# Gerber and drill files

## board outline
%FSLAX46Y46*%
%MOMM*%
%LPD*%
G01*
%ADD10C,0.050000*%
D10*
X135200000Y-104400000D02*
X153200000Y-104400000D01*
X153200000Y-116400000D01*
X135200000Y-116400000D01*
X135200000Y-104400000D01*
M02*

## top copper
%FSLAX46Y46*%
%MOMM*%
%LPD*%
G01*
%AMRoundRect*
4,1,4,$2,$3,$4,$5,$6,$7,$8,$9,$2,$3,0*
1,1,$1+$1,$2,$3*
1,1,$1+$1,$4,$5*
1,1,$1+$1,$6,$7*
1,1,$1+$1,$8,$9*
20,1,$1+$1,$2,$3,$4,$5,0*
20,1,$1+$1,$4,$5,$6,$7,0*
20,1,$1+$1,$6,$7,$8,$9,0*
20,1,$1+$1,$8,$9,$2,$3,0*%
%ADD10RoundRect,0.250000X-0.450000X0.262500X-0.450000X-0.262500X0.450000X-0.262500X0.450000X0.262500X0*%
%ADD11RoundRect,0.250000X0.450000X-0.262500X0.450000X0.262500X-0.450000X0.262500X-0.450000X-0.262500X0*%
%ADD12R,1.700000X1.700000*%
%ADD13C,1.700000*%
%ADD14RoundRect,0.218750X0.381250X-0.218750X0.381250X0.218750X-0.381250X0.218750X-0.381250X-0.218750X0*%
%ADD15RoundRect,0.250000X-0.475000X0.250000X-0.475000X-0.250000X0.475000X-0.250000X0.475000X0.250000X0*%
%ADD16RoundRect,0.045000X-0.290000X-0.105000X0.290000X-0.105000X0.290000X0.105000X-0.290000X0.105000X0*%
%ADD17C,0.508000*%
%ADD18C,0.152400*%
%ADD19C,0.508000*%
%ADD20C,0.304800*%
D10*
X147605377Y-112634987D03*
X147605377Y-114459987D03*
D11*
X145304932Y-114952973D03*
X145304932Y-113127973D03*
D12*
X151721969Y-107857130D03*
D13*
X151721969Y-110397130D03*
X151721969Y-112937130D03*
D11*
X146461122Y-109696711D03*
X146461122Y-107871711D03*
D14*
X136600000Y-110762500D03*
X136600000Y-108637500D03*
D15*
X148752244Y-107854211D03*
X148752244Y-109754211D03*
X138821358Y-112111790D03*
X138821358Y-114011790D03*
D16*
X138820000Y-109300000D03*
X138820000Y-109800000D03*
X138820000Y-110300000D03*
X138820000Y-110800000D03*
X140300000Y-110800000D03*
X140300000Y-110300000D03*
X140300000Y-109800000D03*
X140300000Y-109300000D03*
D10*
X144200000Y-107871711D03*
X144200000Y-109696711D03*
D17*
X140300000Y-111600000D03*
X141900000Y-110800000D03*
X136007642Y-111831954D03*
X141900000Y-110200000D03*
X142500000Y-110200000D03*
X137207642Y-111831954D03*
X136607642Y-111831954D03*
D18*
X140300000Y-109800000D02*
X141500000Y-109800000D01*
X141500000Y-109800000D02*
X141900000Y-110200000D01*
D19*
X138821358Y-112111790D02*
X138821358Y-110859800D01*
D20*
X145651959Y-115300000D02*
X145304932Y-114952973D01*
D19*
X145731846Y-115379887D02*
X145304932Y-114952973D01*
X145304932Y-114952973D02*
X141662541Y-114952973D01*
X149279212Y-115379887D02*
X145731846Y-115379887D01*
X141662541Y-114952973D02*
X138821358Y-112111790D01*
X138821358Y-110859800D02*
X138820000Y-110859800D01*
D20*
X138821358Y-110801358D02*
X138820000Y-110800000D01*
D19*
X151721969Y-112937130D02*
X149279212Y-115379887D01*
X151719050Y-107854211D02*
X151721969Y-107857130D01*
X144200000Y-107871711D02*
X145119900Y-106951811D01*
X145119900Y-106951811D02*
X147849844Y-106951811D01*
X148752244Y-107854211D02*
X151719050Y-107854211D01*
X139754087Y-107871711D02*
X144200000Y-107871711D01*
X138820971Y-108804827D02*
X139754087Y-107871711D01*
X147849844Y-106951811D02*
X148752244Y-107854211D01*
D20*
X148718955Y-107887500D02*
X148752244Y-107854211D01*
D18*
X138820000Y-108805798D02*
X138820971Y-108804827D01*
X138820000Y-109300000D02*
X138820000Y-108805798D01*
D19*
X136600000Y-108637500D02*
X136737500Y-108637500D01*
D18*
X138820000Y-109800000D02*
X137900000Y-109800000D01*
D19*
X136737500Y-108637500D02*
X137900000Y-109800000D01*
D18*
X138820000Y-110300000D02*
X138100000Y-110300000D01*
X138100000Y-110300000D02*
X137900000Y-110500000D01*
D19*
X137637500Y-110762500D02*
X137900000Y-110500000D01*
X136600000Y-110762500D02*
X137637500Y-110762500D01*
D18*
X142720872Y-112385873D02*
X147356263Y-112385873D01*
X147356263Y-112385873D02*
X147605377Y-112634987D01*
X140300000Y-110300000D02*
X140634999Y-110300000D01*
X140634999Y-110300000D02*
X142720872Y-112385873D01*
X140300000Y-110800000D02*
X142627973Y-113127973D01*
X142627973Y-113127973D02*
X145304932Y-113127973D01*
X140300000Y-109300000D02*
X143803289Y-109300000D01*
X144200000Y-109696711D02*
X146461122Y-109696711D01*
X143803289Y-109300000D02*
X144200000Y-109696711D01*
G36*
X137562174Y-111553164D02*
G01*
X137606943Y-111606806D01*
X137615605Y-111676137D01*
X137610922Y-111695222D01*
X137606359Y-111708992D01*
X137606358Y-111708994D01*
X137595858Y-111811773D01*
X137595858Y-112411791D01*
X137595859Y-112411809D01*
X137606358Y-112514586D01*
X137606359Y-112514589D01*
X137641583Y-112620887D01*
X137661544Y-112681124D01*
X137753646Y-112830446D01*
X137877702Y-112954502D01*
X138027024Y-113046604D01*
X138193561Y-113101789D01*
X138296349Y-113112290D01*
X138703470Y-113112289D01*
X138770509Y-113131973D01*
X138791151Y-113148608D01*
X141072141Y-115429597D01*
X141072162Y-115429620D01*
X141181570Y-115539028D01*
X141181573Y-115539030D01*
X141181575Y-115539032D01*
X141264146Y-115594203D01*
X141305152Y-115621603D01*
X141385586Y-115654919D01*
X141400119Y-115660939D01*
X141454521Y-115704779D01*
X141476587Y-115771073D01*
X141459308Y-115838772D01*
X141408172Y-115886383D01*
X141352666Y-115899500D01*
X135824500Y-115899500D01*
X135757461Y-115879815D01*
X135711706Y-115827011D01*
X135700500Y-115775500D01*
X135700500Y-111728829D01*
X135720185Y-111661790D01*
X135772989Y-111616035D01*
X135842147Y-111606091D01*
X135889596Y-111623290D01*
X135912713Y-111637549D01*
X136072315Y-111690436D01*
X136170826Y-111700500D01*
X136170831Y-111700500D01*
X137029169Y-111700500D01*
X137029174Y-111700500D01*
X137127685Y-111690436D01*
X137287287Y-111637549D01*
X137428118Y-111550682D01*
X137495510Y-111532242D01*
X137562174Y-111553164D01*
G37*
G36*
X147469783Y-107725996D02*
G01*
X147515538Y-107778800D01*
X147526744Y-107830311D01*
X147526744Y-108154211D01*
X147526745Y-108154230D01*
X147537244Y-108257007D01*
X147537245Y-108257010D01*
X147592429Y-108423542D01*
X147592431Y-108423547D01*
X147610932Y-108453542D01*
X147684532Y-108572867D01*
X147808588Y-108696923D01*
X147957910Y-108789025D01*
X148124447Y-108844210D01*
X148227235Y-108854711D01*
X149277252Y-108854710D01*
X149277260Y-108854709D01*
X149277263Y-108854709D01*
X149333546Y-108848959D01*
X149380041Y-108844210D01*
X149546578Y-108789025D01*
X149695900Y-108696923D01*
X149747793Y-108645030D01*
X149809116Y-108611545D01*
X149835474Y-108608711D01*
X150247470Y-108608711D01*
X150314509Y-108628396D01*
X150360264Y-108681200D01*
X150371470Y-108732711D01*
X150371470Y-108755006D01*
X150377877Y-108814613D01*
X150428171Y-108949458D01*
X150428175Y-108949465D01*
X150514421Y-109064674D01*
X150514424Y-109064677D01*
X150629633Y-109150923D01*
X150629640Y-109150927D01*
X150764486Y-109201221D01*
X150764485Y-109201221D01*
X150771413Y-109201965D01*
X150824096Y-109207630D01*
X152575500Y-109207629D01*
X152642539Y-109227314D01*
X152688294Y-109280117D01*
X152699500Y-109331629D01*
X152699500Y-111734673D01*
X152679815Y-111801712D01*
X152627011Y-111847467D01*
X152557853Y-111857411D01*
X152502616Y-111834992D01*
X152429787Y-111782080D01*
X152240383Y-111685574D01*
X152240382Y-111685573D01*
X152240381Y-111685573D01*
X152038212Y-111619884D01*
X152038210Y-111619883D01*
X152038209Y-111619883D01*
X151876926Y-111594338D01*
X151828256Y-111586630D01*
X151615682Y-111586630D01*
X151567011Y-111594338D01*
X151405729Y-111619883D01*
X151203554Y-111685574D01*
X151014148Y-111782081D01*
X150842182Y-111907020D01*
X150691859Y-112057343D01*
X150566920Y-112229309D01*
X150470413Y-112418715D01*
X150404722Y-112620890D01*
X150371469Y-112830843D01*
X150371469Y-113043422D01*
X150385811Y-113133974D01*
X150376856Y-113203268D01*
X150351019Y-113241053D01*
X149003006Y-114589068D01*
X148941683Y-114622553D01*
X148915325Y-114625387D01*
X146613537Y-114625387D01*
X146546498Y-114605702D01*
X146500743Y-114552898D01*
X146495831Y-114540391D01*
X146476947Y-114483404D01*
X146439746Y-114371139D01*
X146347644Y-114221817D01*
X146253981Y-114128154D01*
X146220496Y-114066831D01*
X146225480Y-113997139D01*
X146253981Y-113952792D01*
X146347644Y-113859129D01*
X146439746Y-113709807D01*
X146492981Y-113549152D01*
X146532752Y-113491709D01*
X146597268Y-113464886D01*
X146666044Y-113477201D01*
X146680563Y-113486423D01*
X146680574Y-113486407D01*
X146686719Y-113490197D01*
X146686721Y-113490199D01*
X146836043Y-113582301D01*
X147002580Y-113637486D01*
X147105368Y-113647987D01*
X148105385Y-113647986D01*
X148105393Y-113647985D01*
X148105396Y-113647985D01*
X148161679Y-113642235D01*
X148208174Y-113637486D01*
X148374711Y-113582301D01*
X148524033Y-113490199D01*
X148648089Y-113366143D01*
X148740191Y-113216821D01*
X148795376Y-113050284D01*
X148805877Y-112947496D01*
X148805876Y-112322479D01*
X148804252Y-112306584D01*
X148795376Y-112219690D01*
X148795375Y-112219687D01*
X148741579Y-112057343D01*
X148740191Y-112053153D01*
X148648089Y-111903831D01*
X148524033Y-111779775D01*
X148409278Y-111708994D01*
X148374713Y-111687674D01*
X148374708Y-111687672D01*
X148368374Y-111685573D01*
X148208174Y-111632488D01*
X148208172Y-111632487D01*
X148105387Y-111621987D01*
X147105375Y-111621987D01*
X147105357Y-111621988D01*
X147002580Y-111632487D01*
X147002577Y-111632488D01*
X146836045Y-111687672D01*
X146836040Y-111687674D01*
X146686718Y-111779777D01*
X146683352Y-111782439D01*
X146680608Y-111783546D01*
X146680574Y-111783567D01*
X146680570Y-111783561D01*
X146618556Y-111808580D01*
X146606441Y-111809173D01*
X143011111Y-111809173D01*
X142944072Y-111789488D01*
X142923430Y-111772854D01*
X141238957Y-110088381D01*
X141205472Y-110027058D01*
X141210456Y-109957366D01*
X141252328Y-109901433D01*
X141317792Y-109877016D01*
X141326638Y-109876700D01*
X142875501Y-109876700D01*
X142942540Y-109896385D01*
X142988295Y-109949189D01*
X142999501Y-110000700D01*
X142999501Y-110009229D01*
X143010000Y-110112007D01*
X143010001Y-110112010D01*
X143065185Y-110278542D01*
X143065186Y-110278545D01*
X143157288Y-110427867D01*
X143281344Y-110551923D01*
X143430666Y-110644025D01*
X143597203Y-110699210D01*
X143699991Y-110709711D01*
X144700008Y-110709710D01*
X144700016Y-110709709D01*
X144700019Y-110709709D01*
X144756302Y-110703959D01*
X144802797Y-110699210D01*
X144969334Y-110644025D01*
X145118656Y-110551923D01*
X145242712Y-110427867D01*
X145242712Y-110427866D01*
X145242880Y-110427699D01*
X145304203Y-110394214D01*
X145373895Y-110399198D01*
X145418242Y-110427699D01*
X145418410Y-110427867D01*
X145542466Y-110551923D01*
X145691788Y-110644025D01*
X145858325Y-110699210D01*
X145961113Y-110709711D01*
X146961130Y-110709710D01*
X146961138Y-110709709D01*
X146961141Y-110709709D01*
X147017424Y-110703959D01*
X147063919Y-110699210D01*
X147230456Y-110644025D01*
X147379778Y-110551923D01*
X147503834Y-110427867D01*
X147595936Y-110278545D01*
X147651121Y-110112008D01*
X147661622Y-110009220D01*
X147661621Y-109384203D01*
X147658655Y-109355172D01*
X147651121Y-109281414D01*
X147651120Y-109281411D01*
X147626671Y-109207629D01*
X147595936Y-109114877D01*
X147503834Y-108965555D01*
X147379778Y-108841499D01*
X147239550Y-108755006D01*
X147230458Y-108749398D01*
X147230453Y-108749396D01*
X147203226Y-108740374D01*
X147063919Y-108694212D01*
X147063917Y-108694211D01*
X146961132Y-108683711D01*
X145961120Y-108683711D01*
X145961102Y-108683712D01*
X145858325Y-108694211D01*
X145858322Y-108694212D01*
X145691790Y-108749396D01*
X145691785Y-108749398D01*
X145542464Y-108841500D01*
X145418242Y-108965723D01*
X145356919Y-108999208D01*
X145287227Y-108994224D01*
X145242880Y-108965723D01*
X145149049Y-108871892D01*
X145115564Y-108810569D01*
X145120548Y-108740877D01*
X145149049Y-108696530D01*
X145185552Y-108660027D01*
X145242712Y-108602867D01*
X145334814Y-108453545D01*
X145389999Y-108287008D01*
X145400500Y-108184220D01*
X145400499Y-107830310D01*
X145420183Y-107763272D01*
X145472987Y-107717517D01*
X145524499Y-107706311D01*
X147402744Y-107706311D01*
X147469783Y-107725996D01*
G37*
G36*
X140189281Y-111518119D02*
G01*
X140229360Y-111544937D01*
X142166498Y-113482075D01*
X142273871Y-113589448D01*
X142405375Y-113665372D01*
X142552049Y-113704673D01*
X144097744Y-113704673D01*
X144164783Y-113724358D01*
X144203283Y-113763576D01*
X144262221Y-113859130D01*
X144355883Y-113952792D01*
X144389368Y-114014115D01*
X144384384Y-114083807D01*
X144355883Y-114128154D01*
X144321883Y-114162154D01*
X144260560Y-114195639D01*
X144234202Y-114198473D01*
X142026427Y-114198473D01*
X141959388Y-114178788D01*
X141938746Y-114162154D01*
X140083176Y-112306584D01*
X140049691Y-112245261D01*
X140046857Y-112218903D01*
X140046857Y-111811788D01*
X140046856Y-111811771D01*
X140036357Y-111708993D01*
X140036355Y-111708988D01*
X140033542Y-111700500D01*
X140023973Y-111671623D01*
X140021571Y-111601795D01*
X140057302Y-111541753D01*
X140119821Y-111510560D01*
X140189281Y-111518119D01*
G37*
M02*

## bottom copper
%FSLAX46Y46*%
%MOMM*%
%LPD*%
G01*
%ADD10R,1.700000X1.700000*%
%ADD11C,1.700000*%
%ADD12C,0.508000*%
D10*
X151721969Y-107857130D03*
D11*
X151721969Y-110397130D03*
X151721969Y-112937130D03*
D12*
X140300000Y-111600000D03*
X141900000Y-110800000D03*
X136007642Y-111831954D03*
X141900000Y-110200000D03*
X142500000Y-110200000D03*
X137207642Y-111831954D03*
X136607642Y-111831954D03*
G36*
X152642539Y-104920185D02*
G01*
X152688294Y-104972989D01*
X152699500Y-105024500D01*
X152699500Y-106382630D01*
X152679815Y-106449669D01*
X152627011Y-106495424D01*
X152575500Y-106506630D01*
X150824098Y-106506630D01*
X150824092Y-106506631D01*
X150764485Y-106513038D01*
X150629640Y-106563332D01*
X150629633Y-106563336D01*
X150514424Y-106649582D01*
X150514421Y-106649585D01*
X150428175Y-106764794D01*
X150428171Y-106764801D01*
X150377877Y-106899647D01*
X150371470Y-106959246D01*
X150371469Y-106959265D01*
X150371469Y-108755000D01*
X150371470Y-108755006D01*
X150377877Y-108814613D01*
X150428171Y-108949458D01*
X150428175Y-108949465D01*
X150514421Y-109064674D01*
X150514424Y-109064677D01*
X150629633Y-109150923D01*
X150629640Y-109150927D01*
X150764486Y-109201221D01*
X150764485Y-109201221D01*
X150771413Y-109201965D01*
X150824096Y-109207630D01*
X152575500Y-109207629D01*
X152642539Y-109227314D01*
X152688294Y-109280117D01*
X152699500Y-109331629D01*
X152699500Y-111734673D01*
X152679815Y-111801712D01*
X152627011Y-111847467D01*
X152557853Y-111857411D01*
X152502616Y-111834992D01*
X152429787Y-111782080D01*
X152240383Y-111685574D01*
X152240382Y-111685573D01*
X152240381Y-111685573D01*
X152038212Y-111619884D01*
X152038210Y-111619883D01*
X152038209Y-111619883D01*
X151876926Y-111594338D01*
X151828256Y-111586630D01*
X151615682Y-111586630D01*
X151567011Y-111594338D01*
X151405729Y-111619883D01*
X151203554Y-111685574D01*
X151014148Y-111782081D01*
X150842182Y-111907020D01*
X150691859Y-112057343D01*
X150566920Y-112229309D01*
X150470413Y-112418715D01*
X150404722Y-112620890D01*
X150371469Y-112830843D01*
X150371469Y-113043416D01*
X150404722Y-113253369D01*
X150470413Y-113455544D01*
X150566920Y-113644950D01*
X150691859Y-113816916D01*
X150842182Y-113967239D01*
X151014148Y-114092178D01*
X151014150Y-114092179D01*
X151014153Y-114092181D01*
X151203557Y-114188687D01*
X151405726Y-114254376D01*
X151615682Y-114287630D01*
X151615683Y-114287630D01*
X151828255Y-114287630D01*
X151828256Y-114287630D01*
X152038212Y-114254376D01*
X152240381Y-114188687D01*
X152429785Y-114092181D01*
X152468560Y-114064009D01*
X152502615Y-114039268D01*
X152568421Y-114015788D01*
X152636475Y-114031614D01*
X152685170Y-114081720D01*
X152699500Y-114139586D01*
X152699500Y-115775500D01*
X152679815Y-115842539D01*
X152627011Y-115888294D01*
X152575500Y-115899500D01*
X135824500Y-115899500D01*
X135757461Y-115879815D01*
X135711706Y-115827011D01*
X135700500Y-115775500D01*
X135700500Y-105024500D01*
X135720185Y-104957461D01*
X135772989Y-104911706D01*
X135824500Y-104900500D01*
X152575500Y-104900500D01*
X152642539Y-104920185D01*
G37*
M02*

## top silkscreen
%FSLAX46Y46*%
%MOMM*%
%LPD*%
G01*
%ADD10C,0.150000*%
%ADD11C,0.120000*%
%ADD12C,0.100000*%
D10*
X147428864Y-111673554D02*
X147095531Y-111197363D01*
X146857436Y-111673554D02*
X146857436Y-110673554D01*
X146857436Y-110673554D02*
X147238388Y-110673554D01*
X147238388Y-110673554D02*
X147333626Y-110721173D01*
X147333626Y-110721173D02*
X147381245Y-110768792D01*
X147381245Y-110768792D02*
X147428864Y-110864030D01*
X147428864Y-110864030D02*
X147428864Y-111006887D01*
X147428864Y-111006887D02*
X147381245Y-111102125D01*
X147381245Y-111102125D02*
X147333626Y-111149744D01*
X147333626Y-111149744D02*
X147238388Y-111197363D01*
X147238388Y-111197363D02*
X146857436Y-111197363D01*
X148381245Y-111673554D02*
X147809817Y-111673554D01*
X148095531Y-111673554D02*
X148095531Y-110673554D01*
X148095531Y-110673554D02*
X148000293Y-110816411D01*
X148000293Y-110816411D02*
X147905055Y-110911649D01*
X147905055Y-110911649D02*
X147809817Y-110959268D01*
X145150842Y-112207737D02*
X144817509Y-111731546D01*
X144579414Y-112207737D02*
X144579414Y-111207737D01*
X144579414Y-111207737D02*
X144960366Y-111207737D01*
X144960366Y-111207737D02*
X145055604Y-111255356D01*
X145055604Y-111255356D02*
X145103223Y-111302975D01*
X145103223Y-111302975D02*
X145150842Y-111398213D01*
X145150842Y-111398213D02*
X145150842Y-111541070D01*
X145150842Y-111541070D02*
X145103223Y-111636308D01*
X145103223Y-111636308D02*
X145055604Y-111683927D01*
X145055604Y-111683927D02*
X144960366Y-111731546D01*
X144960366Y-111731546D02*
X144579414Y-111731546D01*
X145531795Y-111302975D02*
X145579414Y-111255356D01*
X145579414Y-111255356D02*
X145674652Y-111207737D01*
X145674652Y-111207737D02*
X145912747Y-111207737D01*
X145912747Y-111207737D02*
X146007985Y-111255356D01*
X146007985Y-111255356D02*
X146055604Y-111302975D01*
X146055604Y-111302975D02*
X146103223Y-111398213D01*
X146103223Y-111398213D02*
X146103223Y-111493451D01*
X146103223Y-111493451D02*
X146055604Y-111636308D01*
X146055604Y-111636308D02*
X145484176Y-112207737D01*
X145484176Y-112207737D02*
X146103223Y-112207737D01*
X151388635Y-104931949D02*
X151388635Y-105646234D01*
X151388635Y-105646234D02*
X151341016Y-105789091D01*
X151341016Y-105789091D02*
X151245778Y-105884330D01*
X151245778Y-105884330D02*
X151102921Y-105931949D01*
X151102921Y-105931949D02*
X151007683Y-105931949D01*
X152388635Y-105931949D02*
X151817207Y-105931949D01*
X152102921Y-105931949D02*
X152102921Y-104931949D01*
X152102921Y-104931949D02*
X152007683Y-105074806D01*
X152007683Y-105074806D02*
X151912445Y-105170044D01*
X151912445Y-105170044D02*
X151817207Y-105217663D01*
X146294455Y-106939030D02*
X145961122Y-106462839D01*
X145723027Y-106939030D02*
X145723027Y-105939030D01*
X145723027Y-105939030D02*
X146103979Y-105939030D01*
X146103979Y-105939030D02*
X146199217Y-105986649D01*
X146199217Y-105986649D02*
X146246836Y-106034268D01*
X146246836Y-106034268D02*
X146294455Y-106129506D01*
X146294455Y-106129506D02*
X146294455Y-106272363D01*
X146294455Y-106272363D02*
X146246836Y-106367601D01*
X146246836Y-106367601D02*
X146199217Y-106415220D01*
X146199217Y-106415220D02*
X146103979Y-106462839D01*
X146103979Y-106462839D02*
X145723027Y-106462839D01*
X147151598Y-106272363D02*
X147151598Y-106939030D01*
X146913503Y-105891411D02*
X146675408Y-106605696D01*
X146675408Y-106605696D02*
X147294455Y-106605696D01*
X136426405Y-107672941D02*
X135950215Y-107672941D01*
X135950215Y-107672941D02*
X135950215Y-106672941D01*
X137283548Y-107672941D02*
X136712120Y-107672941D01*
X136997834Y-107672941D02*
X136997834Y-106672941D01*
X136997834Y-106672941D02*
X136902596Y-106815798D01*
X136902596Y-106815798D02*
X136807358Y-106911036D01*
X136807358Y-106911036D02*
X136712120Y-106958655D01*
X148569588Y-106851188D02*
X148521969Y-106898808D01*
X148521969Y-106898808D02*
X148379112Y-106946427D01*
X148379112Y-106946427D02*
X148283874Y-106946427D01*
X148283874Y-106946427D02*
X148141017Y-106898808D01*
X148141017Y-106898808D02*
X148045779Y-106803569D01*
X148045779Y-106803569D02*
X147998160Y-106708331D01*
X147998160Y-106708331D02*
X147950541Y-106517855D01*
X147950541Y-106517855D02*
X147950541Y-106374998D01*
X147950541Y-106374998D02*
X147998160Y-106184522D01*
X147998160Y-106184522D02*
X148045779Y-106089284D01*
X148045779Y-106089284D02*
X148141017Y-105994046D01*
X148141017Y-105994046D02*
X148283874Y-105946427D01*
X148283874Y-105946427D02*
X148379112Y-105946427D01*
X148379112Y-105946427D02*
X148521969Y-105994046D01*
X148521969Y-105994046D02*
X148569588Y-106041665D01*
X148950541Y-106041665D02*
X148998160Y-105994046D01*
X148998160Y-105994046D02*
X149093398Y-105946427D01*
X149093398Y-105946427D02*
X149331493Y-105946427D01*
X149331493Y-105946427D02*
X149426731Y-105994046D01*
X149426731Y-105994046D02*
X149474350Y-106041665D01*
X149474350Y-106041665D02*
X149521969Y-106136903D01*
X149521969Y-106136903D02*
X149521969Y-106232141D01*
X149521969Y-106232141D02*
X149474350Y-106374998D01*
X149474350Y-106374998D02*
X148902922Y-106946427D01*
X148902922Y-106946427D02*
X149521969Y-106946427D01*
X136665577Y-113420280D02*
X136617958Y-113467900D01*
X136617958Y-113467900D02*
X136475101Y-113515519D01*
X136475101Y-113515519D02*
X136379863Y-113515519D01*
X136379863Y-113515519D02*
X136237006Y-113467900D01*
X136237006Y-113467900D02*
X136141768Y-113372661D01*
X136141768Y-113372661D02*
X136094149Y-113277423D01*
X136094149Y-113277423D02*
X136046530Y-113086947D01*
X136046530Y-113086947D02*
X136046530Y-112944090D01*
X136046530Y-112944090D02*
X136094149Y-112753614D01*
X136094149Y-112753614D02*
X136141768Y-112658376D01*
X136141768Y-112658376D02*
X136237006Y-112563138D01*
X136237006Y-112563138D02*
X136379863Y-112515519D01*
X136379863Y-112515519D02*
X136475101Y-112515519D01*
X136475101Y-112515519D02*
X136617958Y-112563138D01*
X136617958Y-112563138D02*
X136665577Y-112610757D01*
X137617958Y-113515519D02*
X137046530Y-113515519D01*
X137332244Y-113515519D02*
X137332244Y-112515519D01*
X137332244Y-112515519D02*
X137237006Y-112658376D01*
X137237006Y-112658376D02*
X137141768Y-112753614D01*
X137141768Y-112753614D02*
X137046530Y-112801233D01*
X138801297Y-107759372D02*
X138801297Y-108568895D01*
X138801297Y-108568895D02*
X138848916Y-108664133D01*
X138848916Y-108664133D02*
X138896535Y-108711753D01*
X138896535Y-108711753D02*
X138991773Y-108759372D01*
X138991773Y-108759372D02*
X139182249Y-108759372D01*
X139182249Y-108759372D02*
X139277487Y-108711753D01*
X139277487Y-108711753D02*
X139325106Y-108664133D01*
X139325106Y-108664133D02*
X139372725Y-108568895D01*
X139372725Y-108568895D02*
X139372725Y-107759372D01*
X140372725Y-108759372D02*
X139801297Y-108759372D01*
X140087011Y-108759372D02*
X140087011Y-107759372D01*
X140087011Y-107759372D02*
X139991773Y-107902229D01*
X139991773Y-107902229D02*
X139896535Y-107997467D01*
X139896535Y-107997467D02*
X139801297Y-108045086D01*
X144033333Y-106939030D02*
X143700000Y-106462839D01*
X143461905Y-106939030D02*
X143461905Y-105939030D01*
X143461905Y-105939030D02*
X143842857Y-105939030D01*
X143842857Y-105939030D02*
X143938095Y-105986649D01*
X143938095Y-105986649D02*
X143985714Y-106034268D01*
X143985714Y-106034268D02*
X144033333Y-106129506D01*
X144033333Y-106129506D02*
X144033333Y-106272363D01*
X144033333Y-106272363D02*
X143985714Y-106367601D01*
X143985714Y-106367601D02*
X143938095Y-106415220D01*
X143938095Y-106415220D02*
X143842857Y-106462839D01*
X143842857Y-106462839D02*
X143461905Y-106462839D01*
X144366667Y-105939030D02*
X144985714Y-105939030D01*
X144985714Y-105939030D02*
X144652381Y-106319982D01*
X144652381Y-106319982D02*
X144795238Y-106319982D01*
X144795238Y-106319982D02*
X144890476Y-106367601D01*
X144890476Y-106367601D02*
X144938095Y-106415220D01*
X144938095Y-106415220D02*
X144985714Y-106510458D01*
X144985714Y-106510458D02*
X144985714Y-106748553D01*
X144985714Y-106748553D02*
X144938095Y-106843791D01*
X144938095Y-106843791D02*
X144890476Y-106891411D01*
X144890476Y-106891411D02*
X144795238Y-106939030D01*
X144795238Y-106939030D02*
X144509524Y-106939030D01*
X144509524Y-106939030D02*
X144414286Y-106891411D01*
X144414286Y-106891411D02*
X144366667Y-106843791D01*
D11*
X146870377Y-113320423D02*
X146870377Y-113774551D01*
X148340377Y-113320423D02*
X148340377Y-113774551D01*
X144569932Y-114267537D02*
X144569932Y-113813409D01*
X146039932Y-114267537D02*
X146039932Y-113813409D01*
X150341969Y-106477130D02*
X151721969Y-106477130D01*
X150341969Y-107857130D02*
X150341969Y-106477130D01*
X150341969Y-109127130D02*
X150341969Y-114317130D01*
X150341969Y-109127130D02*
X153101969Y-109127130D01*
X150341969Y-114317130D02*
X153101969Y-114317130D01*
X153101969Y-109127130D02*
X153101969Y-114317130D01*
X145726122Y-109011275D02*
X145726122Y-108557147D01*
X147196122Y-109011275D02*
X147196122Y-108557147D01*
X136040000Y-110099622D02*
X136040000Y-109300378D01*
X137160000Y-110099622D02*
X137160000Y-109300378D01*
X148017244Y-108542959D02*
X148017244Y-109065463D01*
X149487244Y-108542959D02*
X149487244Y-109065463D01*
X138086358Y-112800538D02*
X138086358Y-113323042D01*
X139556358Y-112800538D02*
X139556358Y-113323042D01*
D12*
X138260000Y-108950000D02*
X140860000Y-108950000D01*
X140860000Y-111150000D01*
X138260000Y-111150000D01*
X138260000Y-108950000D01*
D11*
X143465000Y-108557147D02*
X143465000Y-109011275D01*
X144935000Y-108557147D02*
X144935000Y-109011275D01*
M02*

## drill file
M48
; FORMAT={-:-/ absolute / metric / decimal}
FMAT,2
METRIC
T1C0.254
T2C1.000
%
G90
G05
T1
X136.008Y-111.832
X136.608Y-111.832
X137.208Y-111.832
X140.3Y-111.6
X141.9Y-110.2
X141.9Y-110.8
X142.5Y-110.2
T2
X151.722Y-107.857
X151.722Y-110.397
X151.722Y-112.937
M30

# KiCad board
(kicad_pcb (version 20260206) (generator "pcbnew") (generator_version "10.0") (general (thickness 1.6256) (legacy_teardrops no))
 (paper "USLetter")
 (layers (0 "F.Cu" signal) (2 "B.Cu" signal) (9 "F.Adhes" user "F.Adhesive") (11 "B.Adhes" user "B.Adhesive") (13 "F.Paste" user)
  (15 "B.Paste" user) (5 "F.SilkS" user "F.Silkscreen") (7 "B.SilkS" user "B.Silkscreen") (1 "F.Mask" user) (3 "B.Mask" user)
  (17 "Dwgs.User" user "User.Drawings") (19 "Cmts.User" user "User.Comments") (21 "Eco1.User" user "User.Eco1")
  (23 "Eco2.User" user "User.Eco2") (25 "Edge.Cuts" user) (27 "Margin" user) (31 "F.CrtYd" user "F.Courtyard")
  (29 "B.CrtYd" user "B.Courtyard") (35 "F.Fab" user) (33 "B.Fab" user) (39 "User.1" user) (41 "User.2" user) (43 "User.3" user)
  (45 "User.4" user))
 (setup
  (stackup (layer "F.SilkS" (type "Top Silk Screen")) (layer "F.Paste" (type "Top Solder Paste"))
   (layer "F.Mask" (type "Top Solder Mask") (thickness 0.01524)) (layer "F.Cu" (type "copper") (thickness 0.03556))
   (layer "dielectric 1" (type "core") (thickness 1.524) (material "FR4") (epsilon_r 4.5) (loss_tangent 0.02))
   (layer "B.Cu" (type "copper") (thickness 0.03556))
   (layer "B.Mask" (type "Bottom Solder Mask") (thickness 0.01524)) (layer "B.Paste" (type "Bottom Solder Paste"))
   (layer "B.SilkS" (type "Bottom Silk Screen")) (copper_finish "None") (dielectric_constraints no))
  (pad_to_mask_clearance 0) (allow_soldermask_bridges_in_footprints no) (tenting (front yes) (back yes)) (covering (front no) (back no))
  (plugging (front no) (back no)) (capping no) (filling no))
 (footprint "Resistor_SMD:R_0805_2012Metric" (layer "F.Cu") (at 147.605377 113.547487 -90)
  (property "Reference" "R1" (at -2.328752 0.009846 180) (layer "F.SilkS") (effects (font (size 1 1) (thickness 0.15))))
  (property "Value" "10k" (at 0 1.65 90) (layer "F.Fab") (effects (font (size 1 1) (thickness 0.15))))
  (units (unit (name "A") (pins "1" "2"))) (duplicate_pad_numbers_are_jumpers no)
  (fp_line (start -0.227064 0.735) (end 0.227064 0.735) (stroke (width 0.12) (type solid)) (layer "F.SilkS"))
  (fp_line (start -0.227064 -0.735) (end 0.227064 -0.735) (stroke (width 0.12) (type solid)) (layer "F.SilkS"))
  (pad "1" smd roundrect (at -0.9125 0 270) (size 1.025 1.4) (layers "F.Cu" "F.Mask" "F.Paste") (roundrect_rratio 0.243902)
   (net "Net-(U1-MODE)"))
  (pad "2" smd roundrect (at 0.9125 0 270) (size 1.025 1.4) (layers "F.Cu" "F.Mask" "F.Paste") (roundrect_rratio 0.243902) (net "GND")))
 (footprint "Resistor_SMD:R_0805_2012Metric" (layer "F.Cu") (at 145.304932 114.040473 90)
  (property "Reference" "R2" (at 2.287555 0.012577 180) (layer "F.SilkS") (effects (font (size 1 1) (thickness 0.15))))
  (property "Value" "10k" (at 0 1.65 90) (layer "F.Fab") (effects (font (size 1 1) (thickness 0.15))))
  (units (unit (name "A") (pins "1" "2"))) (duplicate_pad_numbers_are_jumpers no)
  (fp_line (start -0.227064 -0.735) (end 0.227064 -0.735) (stroke (width 0.12) (type solid)) (layer "F.SilkS"))
  (fp_line (start -0.227064 0.735) (end 0.227064 0.735) (stroke (width 0.12) (type solid)) (layer "F.SilkS"))
  (pad "1" smd roundrect (at -0.9125 0 90) (size 1.025 1.4) (layers "F.Cu" "F.Mask" "F.Paste") (roundrect_rratio 0.243902) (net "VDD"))
  (pad "2" smd roundrect (at 0.9125 0 90) (size 1.025 1.4) (layers "F.Cu" "F.Mask" "F.Paste") (roundrect_rratio 0.243902)
   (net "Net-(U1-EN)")))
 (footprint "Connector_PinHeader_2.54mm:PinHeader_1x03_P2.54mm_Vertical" (layer "F.Cu") (at 151.721969 107.85713)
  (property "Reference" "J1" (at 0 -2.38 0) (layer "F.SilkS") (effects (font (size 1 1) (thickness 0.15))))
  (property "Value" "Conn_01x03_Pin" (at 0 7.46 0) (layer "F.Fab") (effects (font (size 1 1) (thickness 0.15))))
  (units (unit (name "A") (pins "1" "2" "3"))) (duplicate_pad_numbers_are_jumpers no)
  (fp_line (start -1.38 -1.38) (end 0 -1.38) (stroke (width 0.12) (type solid)) (layer "F.SilkS"))
  (fp_line (start -1.38 0) (end -1.38 -1.38) (stroke (width 0.12) (type solid)) (layer "F.SilkS"))
  (fp_line (start -1.38 1.27) (end -1.38 6.46) (stroke (width 0.12) (type solid)) (layer "F.SilkS"))
  (fp_line (start -1.38 1.27) (end 1.38 1.27) (stroke (width 0.12) (type solid)) (layer "F.SilkS"))
  (fp_line (start -1.38 6.46) (end 1.38 6.46) (stroke (width 0.12) (type solid)) (layer "F.SilkS"))
  (fp_line (start 1.38 1.27) (end 1.38 6.46) (stroke (width 0.12) (type solid)) (layer "F.SilkS"))
  (pad "1" thru_hole rect (at 0 0) (size 1.7 1.7) (drill 1) (layers "*.Cu" "*.Mask") (remove_unused_layers no) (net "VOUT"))
  (pad "2" thru_hole circle (at 0 2.54) (size 1.7 1.7) (drill 1) (layers "*.Cu" "*.Mask") (remove_unused_layers no) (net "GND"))
  (pad "3" thru_hole circle (at 0 5.08) (size 1.7 1.7) (drill 1) (layers "*.Cu" "*.Mask") (remove_unused_layers no) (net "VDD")))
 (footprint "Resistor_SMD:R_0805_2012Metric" (layer "F.Cu") (at 146.461122 108.784211 90)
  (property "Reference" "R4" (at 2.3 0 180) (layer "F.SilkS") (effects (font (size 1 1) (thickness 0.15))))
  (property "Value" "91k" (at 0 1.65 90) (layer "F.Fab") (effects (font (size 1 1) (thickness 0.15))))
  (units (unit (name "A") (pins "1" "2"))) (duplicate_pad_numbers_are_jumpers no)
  (fp_line (start -0.227064 -0.735) (end 0.227064 -0.735) (stroke (width 0.12) (type solid)) (layer "F.SilkS"))
  (fp_line (start -0.227064 0.735) (end 0.227064 0.735) (stroke (width 0.12) (type solid)) (layer "F.SilkS"))
  (pad "1" smd roundrect (at -0.9125 0 90) (size 1.025 1.4) (layers "F.Cu" "F.Mask" "F.Paste") (roundrect_rratio 0.243902)
   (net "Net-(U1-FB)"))
  (pad "2" smd roundrect (at 0.9125 0 90) (size 1.025 1.4) (layers "F.Cu" "F.Mask" "F.Paste") (roundrect_rratio 0.243902) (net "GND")))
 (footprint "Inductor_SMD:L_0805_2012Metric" (layer "F.Cu") (at 136.6 109.7 90)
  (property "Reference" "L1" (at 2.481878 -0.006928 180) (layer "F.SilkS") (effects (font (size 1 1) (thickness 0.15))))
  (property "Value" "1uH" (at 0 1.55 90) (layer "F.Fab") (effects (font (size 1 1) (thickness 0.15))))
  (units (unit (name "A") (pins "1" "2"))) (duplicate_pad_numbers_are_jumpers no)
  (fp_line (start -0.399622 -0.56) (end 0.399622 -0.56) (stroke (width 0.12) (type solid)) (layer "F.SilkS"))
  (fp_line (start -0.399622 0.56) (end 0.399622 0.56) (stroke (width 0.12) (type solid)) (layer "F.SilkS"))
  (pad "1" smd roundrect (at -1.0625 0 90) (size 0.875 1.2) (layers "F.Cu" "F.Mask" "F.Paste") (roundrect_rratio 0.25) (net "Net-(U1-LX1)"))
  (pad "2" smd roundrect (at 1.0625 0 90) (size 0.875 1.2) (layers "F.Cu" "F.Mask" "F.Paste") (roundrect_rratio 0.25) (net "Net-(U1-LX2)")))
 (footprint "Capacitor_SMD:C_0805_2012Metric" (layer "F.Cu") (at 148.752244 108.804211 -90)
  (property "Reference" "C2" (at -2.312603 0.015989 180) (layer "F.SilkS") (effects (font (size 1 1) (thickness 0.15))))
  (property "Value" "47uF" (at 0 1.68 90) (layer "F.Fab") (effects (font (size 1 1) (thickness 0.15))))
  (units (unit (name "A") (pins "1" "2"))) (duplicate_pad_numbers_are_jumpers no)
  (fp_line (start -0.261252 0.735) (end 0.261252 0.735) (stroke (width 0.12) (type solid)) (layer "F.SilkS"))
  (fp_line (start -0.261252 -0.735) (end 0.261252 -0.735) (stroke (width 0.12) (type solid)) (layer "F.SilkS"))
  (pad "1" smd roundrect (at -0.95 0 270) (size 1 1.45) (layers "F.Cu" "F.Mask" "F.Paste") (roundrect_rratio 0.25) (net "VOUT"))
  (pad "2" smd roundrect (at 0.95 0 270) (size 1 1.45) (layers "F.Cu" "F.Mask" "F.Paste") (roundrect_rratio 0.25) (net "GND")))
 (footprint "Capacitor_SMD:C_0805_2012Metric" (layer "F.Cu") (at 138.821358 113.06179 -90)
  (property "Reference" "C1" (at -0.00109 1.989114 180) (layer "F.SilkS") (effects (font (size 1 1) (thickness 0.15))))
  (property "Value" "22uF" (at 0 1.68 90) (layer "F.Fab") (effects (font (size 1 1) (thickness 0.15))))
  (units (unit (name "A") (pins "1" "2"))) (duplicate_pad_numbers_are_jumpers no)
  (fp_line (start -0.261252 0.735) (end 0.261252 0.735) (stroke (width 0.12) (type solid)) (layer "F.SilkS"))
  (fp_line (start -0.261252 -0.735) (end 0.261252 -0.735) (stroke (width 0.12) (type solid)) (layer "F.SilkS"))
  (pad "1" smd roundrect (at -0.95 0 270) (size 1 1.45) (layers "F.Cu" "F.Mask" "F.Paste") (roundrect_rratio 0.25) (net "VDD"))
  (pad "2" smd roundrect (at 0.95 0 270) (size 1 1.45) (layers "F.Cu" "F.Mask" "F.Paste") (roundrect_rratio 0.25) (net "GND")))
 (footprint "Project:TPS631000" (layer "F.Cu") (at 139.56 110.05)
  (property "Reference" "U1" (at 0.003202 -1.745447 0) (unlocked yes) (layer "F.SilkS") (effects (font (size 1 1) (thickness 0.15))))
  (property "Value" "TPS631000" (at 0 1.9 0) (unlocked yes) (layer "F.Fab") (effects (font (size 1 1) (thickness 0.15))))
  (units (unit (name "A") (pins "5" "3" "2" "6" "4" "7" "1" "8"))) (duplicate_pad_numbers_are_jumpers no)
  (fp_rect (start -1.3 -1.1) (end 1.3 1.1) (stroke (width 0.1) (type default)) (fill no) (layer "F.SilkS"))
  (pad "1" smd roundrect (at -0.74 -0.75) (size 0.67 0.3) (layers "F.Cu" "F.Mask" "F.Paste") (roundrect_rratio 0.15) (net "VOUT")
   (solder_mask_margin 0.05) (solder_paste_margin_ratio -0.1))
  (pad "2" smd roundrect (at -0.74 -0.25) (size 0.67 0.3) (layers "F.Cu" "F.Mask" "F.Paste") (roundrect_rratio 0.15) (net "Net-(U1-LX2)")
   (solder_mask_margin 0.05) (solder_paste_margin_ratio -0.1))
  (pad "3" smd roundrect (at -0.74 0.25) (size 0.67 0.3) (layers "F.Cu" "F.Mask" "F.Paste") (roundrect_rratio 0.15) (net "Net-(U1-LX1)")
   (solder_mask_margin 0.05) (solder_paste_margin_ratio -0.1))
  (pad "4" smd roundrect (at -0.74 0.75) (size 0.67 0.3) (layers "F.Cu" "F.Mask" "F.Paste") (roundrect_rratio 0.15) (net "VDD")
   (solder_mask_margin 0.05) (solder_paste_margin_ratio -0.1))
  (pad "5" smd roundrect (at 0.74 0.75) (size 0.67 0.3) (layers "F.Cu" "F.Mask" "F.Paste") (roundrect_rratio 0.15) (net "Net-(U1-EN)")
   (solder_mask_margin 0.05) (solder_paste_margin_ratio -0.1))
  (pad "6" smd roundrect (at 0.74 0.25) (size 0.67 0.3) (layers "F.Cu" "F.Mask" "F.Paste") (roundrect_rratio 0.15) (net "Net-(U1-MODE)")
   (solder_mask_margin 0.05) (solder_paste_margin_ratio -0.1))
  (pad "7" smd roundrect (at 0.74 -0.25) (size 0.67 0.3) (layers "F.Cu" "F.Mask" "F.Paste") (roundrect_rratio 0.15) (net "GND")
   (solder_mask_margin 0.05) (solder_paste_margin_ratio -0.1))
  (pad "8" smd roundrect (at 0.74 -0.75) (size 0.67 0.3) (layers "F.Cu" "F.Mask" "F.Paste") (roundrect_rratio 0.15) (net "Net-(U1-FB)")
   (solder_mask_margin 0.05) (solder_paste_margin_ratio -0.1))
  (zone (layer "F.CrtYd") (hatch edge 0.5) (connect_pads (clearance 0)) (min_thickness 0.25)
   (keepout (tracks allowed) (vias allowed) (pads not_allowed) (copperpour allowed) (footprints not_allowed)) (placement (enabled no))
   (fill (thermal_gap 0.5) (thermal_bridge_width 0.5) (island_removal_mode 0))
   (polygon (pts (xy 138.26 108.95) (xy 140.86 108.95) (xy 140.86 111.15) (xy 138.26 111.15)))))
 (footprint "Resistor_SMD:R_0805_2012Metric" (layer "F.Cu") (at 144.2 108.784211 -90)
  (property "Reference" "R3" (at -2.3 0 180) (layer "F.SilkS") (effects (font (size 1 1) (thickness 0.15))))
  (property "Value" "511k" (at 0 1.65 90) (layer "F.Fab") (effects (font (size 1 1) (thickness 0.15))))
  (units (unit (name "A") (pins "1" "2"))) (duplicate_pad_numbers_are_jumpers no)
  (fp_line (start -0.227064 0.735) (end 0.227064 0.735) (stroke (width 0.12) (type solid)) (layer "F.SilkS"))
  (fp_line (start -0.227064 -0.735) (end 0.227064 -0.735) (stroke (width 0.12) (type solid)) (layer "F.SilkS"))
  (pad "1" smd roundrect (at -0.9125 0 270) (size 1.025 1.4) (layers "F.Cu" "F.Mask" "F.Paste") (roundrect_rratio 0.243902) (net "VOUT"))
  (pad "2" smd roundrect (at 0.9125 0 270) (size 1.025 1.4) (layers "F.Cu" "F.Mask" "F.Paste") (roundrect_rratio 0.243902)
   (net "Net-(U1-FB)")))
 (gr_rect (start 135.2 104.4) (end 153.2 116.4) (stroke (width 0.05) (type solid)) (fill no) (layer "Edge.Cuts"))
 (segment (start 140.3 109.8) (end 141.5 109.8) (width 0.1524) (layer "F.Cu") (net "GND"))
 (segment (start 141.5 109.8) (end 141.9 110.2) (width 0.1524) (layer "F.Cu") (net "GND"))
 (via (at 140.3 111.6) (size 0.508) (drill 0.254) (layers "F.Cu" "B.Cu") (free yes) (capping no) (covering (front no) (back no))
  (plugging (front no) (back no)) (filling no) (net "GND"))
 (via (at 141.9 110.8) (size 0.508) (drill 0.254) (layers "F.Cu" "B.Cu") (free yes) (capping no) (covering (front no) (back no))
  (plugging (front no) (back no)) (filling no) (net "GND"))
 (via (at 136.007642 111.831954) (size 0.508) (drill 0.254) (layers "F.Cu" "B.Cu") (free yes) (capping no) (covering (front no) (back no))
  (plugging (front no) (back no)) (filling no) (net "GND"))
 (via (at 141.9 110.2) (size 0.508) (drill 0.254) (layers "F.Cu" "B.Cu") (free yes) (capping no) (covering (front no) (back no))
  (plugging (front no) (back no)) (filling no) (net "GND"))
 (via (at 142.5 110.2) (size 0.508) (drill 0.254) (layers "F.Cu" "B.Cu") (free yes) (capping no) (covering (front no) (back no))
  (plugging (front no) (back no)) (filling no) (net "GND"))
 (via (at 137.207642 111.831954) (size 0.508) (drill 0.254) (layers "F.Cu" "B.Cu") (free yes) (capping no) (covering (front no) (back no))
  (plugging (front no) (back no)) (filling no) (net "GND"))
 (via (at 136.607642 111.831954) (size 0.508) (drill 0.254) (layers "F.Cu" "B.Cu") (free yes) (capping no) (covering (front no) (back no))
  (plugging (front no) (back no)) (filling no) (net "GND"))
 (segment (start 138.821358 112.11179) (end 138.821358 110.8598) (width 0.508) (layer "F.Cu") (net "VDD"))
 (segment (start 145.651959 115.3) (end 145.304932 114.952973) (width 0.3048) (layer "F.Cu") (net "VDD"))
 (segment (start 145.731846 115.379887) (end 145.304932 114.952973) (width 0.508) (layer "F.Cu") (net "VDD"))
 (segment (start 145.304932 114.952973) (end 141.662541 114.952973) (width 0.508) (layer "F.Cu") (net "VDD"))
 (segment (start 149.279212 115.379887) (end 145.731846 115.379887) (width 0.508) (layer "F.Cu") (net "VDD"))
 (segment (start 141.662541 114.952973) (end 138.821358 112.11179) (width 0.508) (layer "F.Cu") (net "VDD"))
 (segment (start 138.821358 110.8598) (end 138.82 110.8598) (width 0.508) (layer "F.Cu") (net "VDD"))
 (segment (start 138.821358 110.801358) (end 138.82 110.8) (width 0.3048) (layer "F.Cu") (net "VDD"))
 (segment (start 151.721969 112.93713) (end 149.279212 115.379887) (width 0.508) (layer "F.Cu") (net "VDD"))
 (segment (start 151.71905 107.854211) (end 151.721969 107.85713) (width 0.508) (layer "F.Cu") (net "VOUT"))
 (segment (start 144.2 107.871711) (end 145.1199 106.951811) (width 0.508) (layer "F.Cu") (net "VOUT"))
 (segment (start 145.1199 106.951811) (end 147.849844 106.951811) (width 0.508) (layer "F.Cu") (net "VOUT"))
 (segment (start 148.752244 107.854211) (end 151.71905 107.854211) (width 0.508) (layer "F.Cu") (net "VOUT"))
 (segment (start 139.754087 107.871711) (end 144.2 107.871711) (width 0.508) (layer "F.Cu") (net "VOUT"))
 (segment (start 138.820971 108.804827) (end 139.754087 107.871711) (width 0.508) (layer "F.Cu") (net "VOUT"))
 (segment (start 147.849844 106.951811) (end 148.752244 107.854211) (width 0.508) (layer "F.Cu") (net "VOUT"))
 (segment (start 148.718955 107.8875) (end 148.752244 107.854211) (width 0.3048) (layer "F.Cu") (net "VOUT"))
 (segment (start 138.82 108.805798) (end 138.820971 108.804827) (width 0.1524) (layer "F.Cu") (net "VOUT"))
 (segment (start 138.82 109.3) (end 138.82 108.805798) (width 0.1524) (layer "F.Cu") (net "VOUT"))
 (segment (start 136.6 108.6375) (end 136.7375 108.6375) (width 0.508) (layer "F.Cu") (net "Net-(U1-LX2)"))
 (segment (start 138.82 109.8) (end 137.9 109.8) (width 0.1524) (layer "F.Cu") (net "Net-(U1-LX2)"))
 (segment (start 136.7375 108.6375) (end 137.9 109.8) (width 0.508) (layer "F.Cu") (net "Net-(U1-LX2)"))
 (segment (start 138.82 110.3) (end 138.1 110.3) (width 0.1524) (layer "F.Cu") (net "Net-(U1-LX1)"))
 (segment (start 138.1 110.3) (end 137.9 110.5) (width 0.1524) (layer "F.Cu") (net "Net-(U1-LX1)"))
 (segment (start 137.6375 110.7625) (end 137.9 110.5) (width 0.508) (layer "F.Cu") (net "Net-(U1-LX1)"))
 (segment (start 136.6 110.7625) (end 137.6375 110.7625) (width 0.508) (layer "F.Cu") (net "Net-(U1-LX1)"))
 (segment (start 142.720872 112.385873) (end 147.356263 112.385873) (width 0.1524) (layer "F.Cu") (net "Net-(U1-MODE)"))
 (segment (start 147.356263 112.385873) (end 147.605377 112.634987) (width 0.1524) (layer "F.Cu") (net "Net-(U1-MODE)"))
 (segment (start 140.3 110.3) (end 140.634999 110.3) (width 0.1524) (layer "F.Cu") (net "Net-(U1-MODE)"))
 (segment (start 140.634999 110.3) (end 142.720872 112.385873) (width 0.1524) (layer "F.Cu") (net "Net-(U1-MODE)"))
 (segment (start 140.3 110.8) (end 142.627973 113.127973) (width 0.1524) (layer "F.Cu") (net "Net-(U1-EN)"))
 (segment (start 142.627973 113.127973) (end 145.304932 113.127973) (width 0.1524) (layer "F.Cu") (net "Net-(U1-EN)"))
 (segment (start 140.3 109.3) (end 143.803289 109.3) (width 0.1524) (layer "F.Cu") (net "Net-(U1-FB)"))
 (segment (start 144.2 109.696711) (end 146.461122 109.696711) (width 0.1524) (layer "F.Cu") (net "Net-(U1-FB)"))
 (segment (start 143.803289 109.3) (end 144.2 109.696711) (width 0.1524) (layer "F.Cu") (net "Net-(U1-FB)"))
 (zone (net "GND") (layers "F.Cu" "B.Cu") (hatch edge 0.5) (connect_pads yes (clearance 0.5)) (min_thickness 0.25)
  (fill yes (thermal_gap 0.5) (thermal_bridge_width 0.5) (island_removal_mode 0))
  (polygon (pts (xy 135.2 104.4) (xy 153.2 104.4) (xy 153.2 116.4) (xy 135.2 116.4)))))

